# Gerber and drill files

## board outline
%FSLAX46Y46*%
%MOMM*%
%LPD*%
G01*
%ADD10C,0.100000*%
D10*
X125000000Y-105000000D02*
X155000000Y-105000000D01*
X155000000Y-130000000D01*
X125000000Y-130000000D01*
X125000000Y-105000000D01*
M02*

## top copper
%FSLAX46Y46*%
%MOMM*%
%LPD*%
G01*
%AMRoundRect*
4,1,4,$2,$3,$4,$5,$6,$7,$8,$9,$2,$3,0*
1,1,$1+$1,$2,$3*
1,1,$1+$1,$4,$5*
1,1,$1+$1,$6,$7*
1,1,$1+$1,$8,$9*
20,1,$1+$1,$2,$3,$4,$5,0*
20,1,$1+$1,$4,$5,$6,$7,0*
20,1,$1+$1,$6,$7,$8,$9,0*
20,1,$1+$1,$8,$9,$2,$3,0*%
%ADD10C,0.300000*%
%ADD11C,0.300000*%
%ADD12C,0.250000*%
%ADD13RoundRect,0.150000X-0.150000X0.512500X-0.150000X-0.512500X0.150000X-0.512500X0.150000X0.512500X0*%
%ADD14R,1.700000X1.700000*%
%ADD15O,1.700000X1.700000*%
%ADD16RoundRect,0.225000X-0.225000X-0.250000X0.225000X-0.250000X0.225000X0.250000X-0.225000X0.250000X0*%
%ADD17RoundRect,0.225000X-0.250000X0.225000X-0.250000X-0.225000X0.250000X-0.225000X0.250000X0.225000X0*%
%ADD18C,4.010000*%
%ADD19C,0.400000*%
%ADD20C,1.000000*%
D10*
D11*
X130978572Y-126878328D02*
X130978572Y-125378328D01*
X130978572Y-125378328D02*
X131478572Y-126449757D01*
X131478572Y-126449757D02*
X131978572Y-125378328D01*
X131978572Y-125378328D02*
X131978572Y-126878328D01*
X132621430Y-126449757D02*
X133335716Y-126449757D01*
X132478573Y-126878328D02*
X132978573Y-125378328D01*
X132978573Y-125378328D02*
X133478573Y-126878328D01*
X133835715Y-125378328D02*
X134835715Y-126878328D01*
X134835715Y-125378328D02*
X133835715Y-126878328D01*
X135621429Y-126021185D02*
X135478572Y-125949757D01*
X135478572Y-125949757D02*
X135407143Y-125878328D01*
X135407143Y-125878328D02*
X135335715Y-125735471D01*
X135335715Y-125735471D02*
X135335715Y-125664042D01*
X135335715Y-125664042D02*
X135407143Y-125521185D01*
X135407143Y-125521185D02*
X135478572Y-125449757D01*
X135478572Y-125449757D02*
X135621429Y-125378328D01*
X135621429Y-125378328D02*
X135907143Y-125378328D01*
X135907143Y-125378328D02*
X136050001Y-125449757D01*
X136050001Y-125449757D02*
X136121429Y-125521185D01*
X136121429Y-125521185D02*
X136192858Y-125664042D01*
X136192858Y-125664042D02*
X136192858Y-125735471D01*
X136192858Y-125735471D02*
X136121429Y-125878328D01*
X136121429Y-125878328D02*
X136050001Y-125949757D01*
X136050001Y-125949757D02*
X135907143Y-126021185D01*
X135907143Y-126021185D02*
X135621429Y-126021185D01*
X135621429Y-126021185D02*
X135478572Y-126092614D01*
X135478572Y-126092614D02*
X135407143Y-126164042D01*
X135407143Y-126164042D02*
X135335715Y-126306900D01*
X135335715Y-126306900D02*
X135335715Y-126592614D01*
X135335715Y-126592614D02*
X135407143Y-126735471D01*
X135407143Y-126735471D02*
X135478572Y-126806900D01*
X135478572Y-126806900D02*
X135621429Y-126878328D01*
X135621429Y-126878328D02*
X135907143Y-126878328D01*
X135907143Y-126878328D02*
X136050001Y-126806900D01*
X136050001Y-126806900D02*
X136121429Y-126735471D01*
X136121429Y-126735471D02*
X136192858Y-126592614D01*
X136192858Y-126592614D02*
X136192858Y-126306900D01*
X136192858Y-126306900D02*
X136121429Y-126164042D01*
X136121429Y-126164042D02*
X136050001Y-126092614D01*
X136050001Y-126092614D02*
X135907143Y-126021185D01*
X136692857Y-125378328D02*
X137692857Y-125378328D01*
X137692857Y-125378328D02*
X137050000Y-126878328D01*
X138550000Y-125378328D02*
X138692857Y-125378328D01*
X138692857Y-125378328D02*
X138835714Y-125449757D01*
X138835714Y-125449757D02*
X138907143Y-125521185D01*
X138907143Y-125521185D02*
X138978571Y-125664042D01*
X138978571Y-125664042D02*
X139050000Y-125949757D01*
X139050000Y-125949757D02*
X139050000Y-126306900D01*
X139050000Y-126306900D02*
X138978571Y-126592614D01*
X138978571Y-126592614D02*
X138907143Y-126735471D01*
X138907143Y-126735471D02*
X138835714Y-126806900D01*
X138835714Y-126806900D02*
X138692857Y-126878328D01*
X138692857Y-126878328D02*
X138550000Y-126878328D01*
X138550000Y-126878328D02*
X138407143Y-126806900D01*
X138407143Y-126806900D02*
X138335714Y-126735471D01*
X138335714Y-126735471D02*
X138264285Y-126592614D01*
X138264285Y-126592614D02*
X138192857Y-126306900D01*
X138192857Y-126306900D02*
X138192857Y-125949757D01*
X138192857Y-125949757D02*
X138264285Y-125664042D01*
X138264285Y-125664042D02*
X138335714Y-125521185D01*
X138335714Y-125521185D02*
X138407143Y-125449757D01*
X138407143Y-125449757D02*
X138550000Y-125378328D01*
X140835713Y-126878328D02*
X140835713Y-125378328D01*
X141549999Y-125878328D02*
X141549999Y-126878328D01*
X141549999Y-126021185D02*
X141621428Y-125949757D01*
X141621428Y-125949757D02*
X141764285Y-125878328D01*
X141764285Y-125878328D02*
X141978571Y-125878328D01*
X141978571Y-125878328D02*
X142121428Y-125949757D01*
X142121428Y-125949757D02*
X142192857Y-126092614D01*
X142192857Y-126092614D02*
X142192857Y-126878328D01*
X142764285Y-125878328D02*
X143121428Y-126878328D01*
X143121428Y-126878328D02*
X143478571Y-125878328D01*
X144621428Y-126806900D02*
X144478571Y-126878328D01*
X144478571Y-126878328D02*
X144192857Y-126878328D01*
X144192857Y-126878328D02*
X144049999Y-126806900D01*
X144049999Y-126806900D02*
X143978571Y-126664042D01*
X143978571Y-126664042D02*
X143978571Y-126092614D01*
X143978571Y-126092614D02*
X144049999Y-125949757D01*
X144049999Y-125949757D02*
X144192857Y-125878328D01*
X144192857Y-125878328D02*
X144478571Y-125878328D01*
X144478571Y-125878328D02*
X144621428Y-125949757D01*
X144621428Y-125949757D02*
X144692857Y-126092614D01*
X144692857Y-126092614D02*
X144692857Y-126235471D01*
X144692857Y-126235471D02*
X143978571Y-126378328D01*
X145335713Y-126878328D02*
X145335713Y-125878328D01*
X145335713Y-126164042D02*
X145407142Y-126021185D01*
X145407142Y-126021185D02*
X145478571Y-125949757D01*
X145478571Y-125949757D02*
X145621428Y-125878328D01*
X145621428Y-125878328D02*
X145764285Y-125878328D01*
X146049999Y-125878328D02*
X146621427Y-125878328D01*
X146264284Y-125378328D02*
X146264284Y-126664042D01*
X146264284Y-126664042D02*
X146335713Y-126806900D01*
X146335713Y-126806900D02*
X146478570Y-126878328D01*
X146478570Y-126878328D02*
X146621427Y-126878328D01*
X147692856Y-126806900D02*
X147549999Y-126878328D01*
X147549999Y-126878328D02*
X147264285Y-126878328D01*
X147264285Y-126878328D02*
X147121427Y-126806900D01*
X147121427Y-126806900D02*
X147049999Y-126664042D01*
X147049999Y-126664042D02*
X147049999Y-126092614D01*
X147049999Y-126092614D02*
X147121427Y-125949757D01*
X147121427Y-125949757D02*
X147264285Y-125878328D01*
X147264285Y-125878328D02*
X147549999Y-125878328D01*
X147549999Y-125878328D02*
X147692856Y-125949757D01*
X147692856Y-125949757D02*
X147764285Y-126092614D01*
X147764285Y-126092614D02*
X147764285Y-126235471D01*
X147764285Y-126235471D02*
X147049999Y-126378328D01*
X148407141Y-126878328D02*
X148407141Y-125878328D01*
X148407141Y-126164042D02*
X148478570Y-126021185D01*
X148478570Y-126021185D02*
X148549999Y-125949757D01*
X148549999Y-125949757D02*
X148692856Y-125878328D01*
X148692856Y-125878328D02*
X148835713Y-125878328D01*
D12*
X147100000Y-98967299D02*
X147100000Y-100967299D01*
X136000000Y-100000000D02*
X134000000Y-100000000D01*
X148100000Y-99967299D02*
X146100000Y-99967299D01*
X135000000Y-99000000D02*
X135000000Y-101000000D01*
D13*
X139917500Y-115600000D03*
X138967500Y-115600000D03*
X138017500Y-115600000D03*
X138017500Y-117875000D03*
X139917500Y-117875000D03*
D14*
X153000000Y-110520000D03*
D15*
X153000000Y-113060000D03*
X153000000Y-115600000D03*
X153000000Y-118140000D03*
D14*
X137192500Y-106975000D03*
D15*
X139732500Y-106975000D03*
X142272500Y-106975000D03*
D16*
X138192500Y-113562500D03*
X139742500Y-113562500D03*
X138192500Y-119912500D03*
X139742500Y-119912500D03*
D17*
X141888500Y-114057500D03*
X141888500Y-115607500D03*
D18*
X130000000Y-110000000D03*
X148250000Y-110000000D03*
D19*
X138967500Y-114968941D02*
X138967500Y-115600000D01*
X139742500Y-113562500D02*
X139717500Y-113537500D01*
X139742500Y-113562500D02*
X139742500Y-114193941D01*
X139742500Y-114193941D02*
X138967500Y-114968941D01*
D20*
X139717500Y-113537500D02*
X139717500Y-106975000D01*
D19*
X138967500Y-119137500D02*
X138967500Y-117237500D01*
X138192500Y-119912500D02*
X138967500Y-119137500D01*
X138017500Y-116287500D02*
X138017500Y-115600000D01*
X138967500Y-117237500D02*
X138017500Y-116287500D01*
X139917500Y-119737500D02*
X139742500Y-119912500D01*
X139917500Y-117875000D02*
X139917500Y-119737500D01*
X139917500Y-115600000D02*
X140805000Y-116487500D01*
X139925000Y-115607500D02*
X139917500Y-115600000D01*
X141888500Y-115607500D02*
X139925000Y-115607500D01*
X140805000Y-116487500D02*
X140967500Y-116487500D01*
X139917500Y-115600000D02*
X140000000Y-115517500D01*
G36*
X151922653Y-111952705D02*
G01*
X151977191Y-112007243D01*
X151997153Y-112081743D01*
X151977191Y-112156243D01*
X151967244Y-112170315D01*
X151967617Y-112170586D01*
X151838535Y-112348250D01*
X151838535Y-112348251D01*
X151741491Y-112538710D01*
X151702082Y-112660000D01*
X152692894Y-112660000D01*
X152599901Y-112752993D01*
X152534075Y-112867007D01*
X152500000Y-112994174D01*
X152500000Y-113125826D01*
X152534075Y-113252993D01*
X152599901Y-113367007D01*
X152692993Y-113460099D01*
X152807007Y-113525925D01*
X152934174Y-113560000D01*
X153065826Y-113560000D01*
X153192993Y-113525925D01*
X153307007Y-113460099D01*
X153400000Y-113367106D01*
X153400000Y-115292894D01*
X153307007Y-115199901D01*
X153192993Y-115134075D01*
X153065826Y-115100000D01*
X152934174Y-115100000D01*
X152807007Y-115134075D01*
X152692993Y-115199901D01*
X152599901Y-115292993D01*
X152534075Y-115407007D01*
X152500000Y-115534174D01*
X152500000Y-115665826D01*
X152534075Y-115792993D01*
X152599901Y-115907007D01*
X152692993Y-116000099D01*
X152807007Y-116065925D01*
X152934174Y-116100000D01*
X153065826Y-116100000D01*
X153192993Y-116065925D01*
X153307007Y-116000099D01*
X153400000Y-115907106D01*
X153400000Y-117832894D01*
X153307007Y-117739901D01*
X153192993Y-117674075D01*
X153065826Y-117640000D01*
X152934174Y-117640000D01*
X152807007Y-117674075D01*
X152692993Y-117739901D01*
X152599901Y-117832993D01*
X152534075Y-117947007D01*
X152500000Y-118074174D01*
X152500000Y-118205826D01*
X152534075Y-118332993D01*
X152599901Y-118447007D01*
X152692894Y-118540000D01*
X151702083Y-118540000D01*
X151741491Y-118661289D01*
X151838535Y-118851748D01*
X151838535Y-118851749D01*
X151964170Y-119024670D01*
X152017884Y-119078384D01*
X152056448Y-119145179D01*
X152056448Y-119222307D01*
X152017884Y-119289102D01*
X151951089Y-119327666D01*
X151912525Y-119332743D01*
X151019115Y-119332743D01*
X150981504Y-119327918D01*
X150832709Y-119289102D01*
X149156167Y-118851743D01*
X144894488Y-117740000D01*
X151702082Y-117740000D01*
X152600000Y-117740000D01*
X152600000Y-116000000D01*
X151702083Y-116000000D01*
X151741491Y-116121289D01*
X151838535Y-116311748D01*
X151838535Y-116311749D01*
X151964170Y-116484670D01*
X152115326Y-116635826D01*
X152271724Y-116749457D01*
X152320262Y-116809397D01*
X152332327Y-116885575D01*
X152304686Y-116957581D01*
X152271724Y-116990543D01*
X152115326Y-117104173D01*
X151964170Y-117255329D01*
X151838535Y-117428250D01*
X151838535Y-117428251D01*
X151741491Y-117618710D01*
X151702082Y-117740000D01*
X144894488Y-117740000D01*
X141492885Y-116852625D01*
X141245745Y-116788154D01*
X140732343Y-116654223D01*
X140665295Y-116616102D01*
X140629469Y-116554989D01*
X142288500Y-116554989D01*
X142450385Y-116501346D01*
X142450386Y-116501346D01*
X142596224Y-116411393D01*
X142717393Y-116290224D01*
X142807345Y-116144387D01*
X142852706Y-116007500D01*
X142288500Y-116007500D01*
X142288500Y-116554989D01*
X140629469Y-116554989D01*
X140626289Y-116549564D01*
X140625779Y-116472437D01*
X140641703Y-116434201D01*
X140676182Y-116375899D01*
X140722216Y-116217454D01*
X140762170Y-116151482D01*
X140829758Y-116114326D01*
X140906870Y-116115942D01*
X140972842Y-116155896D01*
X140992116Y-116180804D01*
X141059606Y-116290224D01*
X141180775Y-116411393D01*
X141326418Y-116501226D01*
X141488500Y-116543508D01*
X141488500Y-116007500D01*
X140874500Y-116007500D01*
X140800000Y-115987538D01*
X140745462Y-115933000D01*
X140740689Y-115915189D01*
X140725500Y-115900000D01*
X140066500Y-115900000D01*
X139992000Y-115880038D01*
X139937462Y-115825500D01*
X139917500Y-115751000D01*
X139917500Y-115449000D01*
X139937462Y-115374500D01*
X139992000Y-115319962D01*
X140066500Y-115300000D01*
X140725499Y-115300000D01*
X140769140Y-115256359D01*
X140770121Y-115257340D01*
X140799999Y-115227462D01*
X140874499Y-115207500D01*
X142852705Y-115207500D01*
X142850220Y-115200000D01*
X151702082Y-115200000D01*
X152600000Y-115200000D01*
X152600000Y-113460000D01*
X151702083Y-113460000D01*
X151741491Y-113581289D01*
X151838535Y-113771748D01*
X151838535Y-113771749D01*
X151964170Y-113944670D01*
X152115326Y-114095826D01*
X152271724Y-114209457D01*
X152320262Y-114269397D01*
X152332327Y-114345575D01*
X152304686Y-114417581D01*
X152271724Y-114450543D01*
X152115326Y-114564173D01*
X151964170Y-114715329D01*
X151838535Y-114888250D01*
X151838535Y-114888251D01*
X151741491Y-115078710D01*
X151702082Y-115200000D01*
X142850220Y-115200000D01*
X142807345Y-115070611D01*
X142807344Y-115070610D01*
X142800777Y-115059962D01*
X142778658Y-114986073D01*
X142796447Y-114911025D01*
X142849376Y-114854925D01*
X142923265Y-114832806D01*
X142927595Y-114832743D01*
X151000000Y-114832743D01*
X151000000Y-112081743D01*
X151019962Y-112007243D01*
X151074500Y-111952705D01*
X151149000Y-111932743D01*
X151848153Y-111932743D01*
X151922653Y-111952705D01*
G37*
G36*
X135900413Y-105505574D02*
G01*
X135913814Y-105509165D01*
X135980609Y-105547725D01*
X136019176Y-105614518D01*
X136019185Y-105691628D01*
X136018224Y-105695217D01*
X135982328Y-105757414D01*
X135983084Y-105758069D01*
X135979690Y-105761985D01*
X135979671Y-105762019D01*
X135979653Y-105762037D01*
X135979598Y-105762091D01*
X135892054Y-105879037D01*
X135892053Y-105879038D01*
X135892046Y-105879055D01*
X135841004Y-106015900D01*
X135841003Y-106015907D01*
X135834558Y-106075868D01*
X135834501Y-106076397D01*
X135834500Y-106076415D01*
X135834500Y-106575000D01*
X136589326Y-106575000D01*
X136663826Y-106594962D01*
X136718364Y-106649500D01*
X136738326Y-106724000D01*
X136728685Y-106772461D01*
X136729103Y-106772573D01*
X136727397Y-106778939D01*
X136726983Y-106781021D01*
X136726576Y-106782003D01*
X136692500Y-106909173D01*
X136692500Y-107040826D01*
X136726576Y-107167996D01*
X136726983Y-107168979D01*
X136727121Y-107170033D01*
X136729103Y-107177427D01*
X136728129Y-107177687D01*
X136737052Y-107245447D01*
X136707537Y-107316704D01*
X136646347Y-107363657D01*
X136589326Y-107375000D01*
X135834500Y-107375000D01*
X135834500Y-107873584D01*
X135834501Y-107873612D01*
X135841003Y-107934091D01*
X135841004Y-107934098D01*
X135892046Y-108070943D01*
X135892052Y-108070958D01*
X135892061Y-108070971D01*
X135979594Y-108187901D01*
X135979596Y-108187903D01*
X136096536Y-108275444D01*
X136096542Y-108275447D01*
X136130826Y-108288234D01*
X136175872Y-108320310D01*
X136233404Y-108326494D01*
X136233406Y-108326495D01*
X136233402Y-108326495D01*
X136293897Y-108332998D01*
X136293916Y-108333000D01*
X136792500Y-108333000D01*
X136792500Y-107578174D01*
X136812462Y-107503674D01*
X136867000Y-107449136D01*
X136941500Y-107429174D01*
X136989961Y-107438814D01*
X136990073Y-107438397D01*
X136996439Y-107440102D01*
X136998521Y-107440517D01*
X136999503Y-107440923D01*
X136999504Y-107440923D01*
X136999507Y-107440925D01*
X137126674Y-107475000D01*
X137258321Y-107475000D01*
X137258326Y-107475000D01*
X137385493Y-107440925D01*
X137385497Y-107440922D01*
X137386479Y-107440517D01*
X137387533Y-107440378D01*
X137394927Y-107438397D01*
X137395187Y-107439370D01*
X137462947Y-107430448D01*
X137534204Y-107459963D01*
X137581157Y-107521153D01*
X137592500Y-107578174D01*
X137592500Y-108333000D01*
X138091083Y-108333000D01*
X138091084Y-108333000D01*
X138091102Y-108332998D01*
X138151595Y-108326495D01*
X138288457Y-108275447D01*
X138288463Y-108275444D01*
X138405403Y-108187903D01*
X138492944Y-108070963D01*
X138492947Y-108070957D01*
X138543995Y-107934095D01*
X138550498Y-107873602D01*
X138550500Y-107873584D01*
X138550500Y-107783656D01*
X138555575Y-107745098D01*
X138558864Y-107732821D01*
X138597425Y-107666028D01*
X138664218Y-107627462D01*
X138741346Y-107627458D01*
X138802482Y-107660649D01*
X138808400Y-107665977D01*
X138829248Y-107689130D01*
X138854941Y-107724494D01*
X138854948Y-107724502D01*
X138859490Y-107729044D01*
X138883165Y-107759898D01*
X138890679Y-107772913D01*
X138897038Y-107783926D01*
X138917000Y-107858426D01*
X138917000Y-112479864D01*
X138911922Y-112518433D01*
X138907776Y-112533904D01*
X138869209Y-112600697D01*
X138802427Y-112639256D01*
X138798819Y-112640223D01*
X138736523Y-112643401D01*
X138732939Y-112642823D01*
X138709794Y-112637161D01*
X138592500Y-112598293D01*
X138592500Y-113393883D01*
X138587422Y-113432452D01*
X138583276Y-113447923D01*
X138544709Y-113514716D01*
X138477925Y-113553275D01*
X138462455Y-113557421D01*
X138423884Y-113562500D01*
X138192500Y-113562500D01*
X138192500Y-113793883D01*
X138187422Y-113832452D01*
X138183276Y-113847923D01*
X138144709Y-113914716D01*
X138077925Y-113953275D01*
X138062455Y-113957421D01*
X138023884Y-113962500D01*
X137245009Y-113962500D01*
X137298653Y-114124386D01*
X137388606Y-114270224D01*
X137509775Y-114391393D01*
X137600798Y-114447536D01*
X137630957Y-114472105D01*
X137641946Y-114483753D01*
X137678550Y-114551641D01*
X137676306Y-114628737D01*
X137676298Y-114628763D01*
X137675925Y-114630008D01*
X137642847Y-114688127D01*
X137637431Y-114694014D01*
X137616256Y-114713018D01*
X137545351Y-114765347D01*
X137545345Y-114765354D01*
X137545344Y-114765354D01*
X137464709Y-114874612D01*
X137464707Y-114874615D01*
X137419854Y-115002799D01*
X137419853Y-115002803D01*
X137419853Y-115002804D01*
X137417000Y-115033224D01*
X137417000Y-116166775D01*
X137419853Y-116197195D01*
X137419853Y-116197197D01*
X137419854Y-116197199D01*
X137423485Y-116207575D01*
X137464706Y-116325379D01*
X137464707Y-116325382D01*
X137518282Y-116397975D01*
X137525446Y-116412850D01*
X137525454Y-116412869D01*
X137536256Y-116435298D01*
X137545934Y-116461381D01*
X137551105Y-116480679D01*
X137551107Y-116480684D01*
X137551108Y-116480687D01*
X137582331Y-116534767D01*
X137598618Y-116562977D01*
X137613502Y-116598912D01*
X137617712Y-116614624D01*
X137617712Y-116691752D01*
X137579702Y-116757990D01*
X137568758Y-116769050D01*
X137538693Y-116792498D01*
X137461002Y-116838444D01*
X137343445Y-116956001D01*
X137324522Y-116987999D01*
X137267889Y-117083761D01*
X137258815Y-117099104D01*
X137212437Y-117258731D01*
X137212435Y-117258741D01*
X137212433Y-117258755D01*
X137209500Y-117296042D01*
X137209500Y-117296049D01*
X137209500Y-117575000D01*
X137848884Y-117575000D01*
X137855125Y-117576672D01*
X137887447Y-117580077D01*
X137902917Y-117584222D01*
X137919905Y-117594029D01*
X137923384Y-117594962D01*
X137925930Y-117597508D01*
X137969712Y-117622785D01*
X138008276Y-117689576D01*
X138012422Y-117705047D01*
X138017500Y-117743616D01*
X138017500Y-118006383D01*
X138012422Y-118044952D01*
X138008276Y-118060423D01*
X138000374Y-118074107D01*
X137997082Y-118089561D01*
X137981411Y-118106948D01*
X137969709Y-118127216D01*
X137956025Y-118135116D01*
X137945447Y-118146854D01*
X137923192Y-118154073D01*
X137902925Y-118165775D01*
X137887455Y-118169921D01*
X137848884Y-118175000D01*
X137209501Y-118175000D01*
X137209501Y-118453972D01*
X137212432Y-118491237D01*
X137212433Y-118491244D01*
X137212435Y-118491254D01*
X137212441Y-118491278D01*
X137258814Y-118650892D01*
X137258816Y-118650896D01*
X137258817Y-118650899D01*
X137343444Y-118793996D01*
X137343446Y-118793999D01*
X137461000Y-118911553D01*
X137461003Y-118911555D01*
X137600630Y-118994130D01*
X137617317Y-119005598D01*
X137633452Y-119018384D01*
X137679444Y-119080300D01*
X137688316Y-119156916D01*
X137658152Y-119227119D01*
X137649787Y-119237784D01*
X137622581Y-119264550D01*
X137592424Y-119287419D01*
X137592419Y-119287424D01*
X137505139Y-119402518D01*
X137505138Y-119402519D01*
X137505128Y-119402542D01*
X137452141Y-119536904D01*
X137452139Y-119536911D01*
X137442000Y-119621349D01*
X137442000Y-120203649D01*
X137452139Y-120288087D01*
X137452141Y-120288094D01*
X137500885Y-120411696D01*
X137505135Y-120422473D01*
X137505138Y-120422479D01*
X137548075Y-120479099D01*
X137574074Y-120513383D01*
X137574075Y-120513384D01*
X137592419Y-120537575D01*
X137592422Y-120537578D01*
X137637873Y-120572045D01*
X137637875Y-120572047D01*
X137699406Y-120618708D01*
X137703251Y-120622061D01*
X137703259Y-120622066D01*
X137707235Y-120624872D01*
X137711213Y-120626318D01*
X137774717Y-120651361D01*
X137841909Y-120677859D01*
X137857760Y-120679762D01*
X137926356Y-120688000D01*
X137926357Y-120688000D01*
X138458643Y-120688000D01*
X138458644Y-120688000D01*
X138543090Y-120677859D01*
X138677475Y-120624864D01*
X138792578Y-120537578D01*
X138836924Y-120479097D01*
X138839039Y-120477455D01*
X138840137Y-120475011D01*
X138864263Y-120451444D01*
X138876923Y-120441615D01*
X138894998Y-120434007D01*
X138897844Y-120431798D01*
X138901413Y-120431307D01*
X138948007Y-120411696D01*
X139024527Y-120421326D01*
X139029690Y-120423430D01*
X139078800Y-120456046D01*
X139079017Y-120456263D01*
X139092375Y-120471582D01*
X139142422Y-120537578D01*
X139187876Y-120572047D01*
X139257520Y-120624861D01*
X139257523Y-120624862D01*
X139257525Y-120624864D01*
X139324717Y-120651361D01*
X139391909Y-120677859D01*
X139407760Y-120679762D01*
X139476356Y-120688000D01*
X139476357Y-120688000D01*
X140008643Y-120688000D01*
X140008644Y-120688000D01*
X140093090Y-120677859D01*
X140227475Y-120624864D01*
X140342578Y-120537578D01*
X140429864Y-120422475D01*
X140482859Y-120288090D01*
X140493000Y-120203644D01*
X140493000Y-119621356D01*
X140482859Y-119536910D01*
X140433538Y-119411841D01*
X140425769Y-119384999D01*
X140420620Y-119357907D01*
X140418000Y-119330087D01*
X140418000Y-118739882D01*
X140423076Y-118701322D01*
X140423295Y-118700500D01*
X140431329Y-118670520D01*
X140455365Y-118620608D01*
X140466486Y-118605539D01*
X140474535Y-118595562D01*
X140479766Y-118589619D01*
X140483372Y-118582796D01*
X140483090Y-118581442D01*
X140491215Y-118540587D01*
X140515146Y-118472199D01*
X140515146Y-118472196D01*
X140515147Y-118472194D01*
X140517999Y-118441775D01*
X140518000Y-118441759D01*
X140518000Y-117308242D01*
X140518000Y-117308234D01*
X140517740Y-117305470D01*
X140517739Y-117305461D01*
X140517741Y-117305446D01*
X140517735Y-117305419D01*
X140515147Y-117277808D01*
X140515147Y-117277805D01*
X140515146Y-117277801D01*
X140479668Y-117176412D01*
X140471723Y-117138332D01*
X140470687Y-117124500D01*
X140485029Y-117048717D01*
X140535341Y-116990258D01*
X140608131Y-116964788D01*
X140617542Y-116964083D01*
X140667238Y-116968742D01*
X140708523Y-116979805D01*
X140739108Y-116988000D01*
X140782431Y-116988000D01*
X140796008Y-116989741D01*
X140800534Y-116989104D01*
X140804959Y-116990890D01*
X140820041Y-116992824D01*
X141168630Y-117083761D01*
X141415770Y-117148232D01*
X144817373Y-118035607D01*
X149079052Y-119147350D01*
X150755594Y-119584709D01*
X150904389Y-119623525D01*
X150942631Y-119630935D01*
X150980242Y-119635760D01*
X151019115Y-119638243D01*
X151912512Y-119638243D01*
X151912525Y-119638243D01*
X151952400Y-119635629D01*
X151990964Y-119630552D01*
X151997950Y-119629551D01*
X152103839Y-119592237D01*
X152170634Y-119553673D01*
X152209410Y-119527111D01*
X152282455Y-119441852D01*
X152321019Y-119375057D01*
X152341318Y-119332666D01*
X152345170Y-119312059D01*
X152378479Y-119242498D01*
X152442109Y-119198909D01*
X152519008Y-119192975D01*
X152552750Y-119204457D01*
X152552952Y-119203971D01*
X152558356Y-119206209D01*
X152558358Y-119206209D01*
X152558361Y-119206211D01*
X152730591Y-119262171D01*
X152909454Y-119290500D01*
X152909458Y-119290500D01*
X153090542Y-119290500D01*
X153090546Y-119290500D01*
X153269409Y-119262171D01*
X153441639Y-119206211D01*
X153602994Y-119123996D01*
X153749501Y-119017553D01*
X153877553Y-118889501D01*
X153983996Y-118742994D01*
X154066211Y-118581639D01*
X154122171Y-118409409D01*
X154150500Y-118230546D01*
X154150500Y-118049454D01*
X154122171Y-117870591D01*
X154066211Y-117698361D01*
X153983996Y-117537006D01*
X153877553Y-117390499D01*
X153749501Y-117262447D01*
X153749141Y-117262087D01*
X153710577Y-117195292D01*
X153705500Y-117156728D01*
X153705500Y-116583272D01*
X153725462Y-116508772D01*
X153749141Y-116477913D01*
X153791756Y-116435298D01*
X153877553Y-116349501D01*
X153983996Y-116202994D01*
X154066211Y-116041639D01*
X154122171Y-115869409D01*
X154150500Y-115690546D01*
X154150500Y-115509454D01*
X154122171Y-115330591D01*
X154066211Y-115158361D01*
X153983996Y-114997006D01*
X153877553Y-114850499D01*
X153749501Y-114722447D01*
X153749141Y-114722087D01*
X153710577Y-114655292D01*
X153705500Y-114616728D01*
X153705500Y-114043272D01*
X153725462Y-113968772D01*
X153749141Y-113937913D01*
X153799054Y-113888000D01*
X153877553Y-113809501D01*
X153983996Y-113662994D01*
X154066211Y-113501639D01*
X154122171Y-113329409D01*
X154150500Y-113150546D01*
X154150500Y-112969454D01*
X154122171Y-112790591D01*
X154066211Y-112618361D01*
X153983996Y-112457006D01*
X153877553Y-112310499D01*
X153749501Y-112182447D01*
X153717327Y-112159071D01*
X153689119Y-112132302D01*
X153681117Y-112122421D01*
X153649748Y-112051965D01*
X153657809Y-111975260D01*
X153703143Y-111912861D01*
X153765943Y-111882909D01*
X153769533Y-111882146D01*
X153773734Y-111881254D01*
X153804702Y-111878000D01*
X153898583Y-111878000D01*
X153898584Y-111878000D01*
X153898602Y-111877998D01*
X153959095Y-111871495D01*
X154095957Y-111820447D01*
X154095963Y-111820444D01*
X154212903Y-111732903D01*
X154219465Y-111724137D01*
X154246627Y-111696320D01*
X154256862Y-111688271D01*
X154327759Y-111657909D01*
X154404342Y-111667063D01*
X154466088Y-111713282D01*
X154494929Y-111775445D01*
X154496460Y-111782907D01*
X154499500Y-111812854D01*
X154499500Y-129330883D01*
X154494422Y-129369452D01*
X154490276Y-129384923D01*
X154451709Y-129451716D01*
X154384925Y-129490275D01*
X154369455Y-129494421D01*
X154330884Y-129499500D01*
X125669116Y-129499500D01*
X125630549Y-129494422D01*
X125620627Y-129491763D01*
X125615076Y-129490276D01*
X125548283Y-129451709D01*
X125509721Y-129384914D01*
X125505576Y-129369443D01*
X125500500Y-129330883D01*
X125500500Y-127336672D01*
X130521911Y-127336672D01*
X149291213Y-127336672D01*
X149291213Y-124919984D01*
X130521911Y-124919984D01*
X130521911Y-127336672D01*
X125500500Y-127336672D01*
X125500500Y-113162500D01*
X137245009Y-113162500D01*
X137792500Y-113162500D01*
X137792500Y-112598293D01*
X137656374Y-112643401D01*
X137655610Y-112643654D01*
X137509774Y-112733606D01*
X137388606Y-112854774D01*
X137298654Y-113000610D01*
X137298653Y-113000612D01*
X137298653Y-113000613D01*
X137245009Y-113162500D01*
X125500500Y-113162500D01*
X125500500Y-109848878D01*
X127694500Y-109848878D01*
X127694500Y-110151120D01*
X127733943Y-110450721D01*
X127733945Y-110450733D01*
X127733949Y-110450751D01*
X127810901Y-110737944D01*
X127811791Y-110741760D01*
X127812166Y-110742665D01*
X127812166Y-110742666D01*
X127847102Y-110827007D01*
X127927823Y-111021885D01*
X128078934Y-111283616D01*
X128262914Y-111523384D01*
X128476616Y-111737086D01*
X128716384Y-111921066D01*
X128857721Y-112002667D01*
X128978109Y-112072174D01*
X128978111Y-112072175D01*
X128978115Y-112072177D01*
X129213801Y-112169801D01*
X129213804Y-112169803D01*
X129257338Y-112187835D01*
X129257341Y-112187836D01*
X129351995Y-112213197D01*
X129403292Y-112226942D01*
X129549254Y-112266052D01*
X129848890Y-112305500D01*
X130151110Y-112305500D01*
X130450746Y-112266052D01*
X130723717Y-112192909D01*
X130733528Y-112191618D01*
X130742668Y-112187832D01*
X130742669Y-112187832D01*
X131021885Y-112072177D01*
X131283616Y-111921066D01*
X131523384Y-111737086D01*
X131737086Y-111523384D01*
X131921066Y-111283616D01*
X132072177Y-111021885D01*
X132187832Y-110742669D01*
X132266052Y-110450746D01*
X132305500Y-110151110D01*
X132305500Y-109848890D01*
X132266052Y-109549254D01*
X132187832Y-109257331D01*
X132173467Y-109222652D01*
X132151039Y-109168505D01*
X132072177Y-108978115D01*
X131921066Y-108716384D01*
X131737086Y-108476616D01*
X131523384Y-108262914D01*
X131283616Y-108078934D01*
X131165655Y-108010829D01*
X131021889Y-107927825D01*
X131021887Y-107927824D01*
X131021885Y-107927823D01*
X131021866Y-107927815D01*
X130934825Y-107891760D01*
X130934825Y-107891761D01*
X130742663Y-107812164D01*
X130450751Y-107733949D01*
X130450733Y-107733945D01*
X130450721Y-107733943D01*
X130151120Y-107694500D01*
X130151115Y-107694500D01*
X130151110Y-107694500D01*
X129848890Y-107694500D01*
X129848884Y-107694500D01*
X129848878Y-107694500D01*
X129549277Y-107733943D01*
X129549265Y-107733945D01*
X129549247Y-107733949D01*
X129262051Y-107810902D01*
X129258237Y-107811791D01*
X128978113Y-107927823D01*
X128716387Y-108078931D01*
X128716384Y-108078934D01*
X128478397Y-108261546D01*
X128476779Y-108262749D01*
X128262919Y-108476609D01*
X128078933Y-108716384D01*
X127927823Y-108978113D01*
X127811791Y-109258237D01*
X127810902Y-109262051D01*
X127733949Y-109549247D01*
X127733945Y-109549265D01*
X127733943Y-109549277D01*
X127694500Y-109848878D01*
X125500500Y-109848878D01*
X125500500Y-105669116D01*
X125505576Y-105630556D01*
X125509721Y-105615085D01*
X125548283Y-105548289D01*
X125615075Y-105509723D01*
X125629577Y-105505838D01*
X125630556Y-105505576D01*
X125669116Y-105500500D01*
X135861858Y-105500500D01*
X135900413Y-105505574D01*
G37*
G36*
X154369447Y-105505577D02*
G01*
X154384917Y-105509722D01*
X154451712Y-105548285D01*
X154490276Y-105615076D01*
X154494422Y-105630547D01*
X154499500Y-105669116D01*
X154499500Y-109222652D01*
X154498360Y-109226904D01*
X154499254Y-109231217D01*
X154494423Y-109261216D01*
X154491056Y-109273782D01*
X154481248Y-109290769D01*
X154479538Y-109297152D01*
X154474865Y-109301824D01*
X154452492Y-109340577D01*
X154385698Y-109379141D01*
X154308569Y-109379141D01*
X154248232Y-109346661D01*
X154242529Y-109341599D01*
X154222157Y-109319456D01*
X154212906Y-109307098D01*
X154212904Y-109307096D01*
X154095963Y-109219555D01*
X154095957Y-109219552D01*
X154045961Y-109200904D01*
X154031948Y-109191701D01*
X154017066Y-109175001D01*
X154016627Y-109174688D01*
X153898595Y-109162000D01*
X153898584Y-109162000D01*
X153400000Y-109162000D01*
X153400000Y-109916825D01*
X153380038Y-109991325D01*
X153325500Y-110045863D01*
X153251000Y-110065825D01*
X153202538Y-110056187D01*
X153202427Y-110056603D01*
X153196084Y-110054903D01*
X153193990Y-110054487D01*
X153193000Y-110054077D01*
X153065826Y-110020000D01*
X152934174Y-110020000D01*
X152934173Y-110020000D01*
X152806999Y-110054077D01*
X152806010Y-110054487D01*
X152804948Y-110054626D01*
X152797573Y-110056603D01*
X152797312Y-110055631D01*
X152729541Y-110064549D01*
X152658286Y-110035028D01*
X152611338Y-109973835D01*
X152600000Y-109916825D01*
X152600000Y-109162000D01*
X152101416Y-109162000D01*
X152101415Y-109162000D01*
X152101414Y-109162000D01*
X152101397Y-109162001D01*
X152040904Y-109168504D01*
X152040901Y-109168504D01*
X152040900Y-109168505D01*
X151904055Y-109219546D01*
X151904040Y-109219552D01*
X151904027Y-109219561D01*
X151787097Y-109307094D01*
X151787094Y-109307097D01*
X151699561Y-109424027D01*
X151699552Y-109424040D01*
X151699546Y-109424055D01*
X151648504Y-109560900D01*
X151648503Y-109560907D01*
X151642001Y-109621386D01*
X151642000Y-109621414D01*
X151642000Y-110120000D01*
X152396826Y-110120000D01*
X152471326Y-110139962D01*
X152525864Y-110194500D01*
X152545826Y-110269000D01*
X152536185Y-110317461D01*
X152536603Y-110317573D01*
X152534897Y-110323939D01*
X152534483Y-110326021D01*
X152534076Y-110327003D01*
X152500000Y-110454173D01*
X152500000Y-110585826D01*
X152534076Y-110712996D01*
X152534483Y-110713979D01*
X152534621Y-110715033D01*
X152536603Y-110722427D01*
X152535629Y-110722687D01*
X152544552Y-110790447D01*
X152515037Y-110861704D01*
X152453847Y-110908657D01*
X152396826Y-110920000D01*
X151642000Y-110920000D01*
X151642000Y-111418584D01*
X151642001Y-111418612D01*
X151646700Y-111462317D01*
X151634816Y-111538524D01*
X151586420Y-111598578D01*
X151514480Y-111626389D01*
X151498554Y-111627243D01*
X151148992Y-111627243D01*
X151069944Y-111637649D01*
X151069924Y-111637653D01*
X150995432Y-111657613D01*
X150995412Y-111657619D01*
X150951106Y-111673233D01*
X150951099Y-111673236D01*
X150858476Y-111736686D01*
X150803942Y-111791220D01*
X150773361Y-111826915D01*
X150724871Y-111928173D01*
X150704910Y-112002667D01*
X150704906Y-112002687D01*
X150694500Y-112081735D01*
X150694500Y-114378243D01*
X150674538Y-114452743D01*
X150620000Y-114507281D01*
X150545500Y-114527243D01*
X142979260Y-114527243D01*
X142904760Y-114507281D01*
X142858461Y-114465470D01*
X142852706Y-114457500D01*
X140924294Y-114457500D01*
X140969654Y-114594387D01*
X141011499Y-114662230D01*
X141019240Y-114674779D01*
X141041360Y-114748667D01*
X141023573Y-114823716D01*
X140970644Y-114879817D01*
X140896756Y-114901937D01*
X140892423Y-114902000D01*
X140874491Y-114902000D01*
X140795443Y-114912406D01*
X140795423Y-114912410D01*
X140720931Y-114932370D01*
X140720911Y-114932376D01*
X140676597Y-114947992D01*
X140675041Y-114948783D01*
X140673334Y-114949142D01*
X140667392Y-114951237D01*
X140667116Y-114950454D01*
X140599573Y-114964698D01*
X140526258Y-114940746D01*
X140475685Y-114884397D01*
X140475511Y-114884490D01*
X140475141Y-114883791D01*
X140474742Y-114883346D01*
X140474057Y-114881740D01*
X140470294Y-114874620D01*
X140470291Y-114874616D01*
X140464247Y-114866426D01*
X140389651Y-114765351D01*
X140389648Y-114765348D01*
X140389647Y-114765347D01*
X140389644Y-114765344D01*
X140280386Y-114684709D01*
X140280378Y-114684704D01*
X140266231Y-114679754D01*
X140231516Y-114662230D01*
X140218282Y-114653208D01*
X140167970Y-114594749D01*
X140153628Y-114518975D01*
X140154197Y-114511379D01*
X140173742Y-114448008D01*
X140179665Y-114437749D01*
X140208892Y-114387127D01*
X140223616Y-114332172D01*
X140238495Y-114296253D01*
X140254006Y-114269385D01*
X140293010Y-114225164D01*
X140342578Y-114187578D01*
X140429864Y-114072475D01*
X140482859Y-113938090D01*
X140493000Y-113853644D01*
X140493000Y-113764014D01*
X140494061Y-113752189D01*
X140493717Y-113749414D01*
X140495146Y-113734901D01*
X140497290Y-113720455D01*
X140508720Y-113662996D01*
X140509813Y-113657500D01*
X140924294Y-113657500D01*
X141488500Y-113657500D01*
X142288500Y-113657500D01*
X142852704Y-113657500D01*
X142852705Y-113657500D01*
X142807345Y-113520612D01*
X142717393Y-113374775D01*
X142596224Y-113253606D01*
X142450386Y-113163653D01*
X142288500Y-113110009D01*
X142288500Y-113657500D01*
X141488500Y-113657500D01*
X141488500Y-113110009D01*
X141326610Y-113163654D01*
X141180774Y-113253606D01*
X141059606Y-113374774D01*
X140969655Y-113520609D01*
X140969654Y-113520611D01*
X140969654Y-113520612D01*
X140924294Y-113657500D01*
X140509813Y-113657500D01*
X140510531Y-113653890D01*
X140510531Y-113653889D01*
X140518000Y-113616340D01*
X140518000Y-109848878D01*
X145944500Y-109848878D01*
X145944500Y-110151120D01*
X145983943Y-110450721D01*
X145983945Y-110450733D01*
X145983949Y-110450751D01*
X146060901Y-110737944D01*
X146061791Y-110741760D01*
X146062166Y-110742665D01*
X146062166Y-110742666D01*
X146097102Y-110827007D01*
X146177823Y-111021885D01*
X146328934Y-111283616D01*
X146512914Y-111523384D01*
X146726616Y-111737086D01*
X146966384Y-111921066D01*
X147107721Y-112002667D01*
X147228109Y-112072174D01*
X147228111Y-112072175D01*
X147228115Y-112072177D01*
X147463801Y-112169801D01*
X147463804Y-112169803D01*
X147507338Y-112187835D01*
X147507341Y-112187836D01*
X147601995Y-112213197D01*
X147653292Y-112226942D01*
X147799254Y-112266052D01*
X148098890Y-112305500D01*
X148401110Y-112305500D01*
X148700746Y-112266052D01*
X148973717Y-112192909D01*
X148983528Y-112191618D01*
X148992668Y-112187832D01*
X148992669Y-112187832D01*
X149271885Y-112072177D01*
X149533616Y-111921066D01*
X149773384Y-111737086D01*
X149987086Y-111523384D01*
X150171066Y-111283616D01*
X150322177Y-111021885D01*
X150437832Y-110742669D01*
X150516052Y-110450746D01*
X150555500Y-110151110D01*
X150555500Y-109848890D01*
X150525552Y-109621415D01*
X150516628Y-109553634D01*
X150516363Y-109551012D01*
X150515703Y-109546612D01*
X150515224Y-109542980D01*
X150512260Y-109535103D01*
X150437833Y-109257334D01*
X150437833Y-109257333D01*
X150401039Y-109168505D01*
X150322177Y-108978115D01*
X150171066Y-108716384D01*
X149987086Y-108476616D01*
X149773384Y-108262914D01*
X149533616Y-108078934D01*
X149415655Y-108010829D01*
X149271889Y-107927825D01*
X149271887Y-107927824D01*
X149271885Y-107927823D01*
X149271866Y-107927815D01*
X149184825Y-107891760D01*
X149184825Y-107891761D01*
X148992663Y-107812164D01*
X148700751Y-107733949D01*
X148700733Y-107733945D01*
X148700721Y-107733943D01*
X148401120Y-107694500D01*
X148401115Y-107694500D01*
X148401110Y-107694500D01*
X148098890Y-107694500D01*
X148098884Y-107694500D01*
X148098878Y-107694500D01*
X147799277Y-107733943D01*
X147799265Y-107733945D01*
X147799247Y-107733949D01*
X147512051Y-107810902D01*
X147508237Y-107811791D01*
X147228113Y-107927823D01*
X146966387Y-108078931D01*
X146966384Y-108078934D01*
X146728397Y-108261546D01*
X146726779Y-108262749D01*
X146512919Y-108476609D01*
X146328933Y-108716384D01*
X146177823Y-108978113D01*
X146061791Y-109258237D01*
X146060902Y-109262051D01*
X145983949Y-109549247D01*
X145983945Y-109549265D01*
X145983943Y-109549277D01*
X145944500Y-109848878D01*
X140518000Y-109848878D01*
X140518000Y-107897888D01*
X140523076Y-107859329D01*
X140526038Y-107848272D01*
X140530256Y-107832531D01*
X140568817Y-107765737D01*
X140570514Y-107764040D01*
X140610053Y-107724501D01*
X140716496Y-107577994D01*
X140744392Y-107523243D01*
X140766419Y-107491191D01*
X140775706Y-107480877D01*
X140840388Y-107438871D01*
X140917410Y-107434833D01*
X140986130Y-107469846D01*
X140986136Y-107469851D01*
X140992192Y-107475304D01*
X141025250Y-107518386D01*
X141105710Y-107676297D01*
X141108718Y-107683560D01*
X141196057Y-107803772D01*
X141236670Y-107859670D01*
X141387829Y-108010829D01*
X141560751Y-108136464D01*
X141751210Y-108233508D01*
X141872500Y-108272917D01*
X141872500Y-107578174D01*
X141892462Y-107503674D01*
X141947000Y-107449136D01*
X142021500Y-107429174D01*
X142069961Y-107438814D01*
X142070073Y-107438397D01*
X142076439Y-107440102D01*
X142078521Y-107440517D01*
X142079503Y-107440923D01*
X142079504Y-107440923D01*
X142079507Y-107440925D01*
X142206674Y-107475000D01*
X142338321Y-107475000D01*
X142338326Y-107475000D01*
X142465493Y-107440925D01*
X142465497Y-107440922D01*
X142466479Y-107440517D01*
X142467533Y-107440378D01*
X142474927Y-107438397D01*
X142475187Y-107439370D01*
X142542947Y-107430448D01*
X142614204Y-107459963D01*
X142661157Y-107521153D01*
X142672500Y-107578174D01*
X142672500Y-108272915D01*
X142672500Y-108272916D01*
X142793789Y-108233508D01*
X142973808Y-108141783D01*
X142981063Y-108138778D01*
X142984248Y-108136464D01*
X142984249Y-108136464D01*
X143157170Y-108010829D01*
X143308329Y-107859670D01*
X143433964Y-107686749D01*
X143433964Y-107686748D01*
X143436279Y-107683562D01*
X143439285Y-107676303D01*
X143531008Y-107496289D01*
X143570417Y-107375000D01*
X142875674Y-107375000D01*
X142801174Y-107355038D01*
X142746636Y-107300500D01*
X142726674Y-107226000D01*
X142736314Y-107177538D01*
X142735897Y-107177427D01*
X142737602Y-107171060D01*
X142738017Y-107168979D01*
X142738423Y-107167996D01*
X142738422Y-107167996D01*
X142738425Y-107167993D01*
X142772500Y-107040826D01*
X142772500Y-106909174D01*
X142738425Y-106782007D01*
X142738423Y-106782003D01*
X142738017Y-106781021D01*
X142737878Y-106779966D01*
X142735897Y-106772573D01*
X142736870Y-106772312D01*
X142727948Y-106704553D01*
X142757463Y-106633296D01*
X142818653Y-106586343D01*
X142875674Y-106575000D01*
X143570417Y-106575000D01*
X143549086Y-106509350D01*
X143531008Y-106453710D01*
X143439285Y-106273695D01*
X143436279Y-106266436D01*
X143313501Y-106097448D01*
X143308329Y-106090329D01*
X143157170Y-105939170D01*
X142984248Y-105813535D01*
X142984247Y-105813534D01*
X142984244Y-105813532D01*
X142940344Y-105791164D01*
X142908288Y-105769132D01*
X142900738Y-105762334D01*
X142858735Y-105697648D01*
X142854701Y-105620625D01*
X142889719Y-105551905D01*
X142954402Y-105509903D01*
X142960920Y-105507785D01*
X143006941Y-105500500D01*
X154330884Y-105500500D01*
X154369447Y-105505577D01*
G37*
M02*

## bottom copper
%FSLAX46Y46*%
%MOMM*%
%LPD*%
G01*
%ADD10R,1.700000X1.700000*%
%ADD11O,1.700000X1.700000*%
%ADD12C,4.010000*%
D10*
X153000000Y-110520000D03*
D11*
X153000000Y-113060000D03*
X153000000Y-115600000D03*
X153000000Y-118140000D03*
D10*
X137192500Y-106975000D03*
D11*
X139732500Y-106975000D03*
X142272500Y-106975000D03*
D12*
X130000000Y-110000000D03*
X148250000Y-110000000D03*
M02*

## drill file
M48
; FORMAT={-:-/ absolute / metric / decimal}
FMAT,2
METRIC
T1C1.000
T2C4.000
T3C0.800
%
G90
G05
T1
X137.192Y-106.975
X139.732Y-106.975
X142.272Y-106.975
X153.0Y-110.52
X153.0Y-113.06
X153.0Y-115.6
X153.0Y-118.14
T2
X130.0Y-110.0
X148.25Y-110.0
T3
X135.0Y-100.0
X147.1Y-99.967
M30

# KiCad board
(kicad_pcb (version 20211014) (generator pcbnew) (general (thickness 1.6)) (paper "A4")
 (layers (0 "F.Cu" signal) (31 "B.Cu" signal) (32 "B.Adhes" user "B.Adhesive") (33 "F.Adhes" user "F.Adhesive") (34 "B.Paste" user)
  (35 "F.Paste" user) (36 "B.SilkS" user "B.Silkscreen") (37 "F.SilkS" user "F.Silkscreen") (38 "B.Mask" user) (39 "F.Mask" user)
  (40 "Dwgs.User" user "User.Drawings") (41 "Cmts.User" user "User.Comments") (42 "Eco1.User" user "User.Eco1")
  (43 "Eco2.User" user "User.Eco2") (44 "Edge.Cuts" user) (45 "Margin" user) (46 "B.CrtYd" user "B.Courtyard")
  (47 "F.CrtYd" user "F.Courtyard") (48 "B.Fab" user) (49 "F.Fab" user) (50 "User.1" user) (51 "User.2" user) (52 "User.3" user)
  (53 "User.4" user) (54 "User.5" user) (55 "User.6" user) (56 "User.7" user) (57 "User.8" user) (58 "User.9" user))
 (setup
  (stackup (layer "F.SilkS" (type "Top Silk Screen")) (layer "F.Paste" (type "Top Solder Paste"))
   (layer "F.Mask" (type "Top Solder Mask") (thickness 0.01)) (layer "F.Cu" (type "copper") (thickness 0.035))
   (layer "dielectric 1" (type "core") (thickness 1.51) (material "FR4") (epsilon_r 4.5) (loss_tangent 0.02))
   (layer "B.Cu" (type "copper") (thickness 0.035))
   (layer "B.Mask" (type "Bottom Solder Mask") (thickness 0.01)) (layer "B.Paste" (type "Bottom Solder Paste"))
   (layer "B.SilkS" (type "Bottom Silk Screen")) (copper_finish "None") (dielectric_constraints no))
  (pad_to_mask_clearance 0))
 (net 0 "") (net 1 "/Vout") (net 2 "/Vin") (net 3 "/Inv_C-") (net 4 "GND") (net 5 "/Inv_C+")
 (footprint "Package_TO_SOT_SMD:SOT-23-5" (layer "F.Cu") (at 138.9675 116.7375 -90) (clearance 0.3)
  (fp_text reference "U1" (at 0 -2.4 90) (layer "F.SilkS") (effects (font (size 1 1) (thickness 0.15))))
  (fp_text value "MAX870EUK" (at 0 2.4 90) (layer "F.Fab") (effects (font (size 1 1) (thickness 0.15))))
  (pad "1" smd roundrect (at -1.1375 -0.95 270) (size 1.325 0.6) (layers "F.Cu" "F.Paste" "F.Mask") (roundrect_rratio 0.25) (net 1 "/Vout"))
  (pad "2" smd roundrect (at -1.1375 0 270) (size 1.325 0.6) (layers "F.Cu" "F.Paste" "F.Mask") (roundrect_rratio 0.25) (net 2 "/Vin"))
  (pad "3" smd roundrect (at -1.1375 0.95 270) (size 1.325 0.6) (layers "F.Cu" "F.Paste" "F.Mask") (roundrect_rratio 0.25) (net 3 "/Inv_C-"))
  (pad "4" smd roundrect (at 1.1375 0.95 270) (size 1.325 0.6) (layers "F.Cu" "F.Paste" "F.Mask") (roundrect_rratio 0.25) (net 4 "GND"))
  (pad "5" smd roundrect (at 1.1375 -0.95 270) (size 1.325 0.6) (layers "F.Cu" "F.Paste" "F.Mask") (roundrect_rratio 0.25) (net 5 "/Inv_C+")))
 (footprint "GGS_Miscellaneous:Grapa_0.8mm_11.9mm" (layer "F.Cu") (at 135 100)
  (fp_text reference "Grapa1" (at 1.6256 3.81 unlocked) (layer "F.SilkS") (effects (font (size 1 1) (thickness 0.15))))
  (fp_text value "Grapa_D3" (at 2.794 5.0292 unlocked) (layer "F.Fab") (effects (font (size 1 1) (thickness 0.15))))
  (fp_line (start 12.1 -1.032701) (end 12.1 0.967299) (layer "F.Cu") (width 0.25))
  (fp_line (start 1 0) (end -1 0) (layer "F.Cu") (width 0.25))
  (fp_line (start 13.1 -0.032701) (end 11.1 -0.032701) (layer "F.Cu") (width 0.25))
  (fp_line (start 0 -1) (end 0 1) (layer "F.Cu") (width 0.25))
  (pad "" np_thru_hole circle (at 12.1 -0.032701) (size 0.8 0.8) (drill 0.8) (layers F&B.Cu *.Mask))
  (pad "" np_thru_hole circle (at 0 0) (size 0.8 0.8) (drill 0.8) (layers F&B.Cu *.Mask)))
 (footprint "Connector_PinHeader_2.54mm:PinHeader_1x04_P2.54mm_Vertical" (layer "F.Cu") (at 153 110.52)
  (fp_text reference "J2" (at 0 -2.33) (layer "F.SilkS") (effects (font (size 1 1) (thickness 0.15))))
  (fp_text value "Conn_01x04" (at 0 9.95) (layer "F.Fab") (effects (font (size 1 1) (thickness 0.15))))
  (pad "1" thru_hole rect (at 0 0) (size 1.7 1.7) (drill 1) (layers *.Cu *.Mask) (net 4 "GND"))
  (pad "2" thru_hole oval (at 0 2.54) (size 1.7 1.7) (drill 1) (layers *.Cu *.Mask) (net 1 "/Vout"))
  (pad "3" thru_hole oval (at 0 5.08) (size 1.7 1.7) (drill 1) (layers *.Cu *.Mask) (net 1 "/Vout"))
  (pad "4" thru_hole oval (at 0 7.62) (size 1.7 1.7) (drill 1) (layers *.Cu *.Mask) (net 1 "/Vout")))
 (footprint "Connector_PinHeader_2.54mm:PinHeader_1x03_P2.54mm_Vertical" (layer "F.Cu") (at 137.1925 106.975 90)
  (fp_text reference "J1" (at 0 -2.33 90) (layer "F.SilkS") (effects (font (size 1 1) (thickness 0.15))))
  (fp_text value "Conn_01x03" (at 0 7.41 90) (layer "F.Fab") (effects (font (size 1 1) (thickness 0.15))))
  (pad "1" thru_hole rect (at 0 0 90) (size 1.7 1.7) (drill 1) (layers *.Cu *.Mask) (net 4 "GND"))
  (pad "2" thru_hole oval (at 0 2.54 90) (size 1.7 1.7) (drill 1) (layers *.Cu *.Mask) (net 2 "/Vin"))
  (pad "3" thru_hole oval (at 0 5.08 90) (size 1.7 1.7) (drill 1) (layers *.Cu *.Mask) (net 4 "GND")))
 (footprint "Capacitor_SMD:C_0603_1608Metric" (layer "F.Cu") (at 138.9675 113.5625)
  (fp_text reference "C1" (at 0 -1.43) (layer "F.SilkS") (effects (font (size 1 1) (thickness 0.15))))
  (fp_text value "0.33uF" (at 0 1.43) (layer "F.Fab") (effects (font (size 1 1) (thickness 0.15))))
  (pad "1" smd roundrect (at -0.775 0) (size 0.9 0.95) (layers "F.Cu" "F.Paste" "F.Mask") (roundrect_rratio 0.25) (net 4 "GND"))
  (pad "2" smd roundrect (at 0.775 0) (size 0.9 0.95) (layers "F.Cu" "F.Paste" "F.Mask") (roundrect_rratio 0.25) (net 2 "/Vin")))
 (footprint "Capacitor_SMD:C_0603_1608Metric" (layer "F.Cu") (at 138.9675 119.9125)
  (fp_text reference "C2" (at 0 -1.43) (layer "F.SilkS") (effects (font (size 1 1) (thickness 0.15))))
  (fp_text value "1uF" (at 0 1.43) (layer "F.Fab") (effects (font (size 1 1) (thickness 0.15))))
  (pad "1" smd roundrect (at -0.775 0) (size 0.9 0.95) (layers "F.Cu" "F.Paste" "F.Mask") (roundrect_rratio 0.25) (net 3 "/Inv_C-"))
  (pad "2" smd roundrect (at 0.775 0) (size 0.9 0.95) (layers "F.Cu" "F.Paste" "F.Mask") (roundrect_rratio 0.25) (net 5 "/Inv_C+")))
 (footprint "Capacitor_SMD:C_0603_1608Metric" (layer "F.Cu") (at 141.8885 114.8325 -90)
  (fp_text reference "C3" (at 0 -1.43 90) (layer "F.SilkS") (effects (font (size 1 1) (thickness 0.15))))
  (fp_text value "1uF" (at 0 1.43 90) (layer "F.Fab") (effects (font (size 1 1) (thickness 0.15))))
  (pad "1" smd roundrect (at -0.775 0 270) (size 0.9 0.95) (layers "F.Cu" "F.Paste" "F.Mask") (roundrect_rratio 0.25) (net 4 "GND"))
  (pad "2" smd roundrect (at 0.775 0 270) (size 0.9 0.95) (layers "F.Cu" "F.Paste" "F.Mask") (roundrect_rratio 0.25) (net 1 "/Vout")))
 (gr_rect (start 125 105) (end 155 130) (layer "Edge.Cuts") (width 0.1) (fill none))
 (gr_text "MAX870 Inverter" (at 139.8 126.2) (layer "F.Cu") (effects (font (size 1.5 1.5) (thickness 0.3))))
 (via (at 130 110) (size 4.01) (drill 4) (layers "F.Cu" "B.Cu") (free) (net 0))
 (via (at 148.25 110) (size 4.01) (drill 4) (layers "F.Cu" "B.Cu") (free) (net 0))
 (segment (start 138.9675 114.968941) (end 138.9675 115.6) (width 0.4) (layer "F.Cu") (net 2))
 (segment (start 139.7425 113.5625) (end 139.7175 113.5375) (width 0.4) (layer "F.Cu") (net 2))
 (segment (start 139.7425 113.5625) (end 139.7425 114.193941) (width 0.4) (layer "F.Cu") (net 2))
 (segment (start 139.7425 114.193941) (end 138.9675 114.968941) (width 0.4) (layer "F.Cu") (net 2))
 (segment (start 139.7175 113.5375) (end 139.7175 106.975) (width 1) (layer "F.Cu") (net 2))
 (segment (start 138.9675 119.1375) (end 138.9675 117.2375) (width 0.4) (layer "F.Cu") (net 3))
 (segment (start 138.1925 119.9125) (end 138.9675 119.1375) (width 0.4) (layer "F.Cu") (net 3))
 (segment (start 138.0175 116.2875) (end 138.0175 115.6) (width 0.4) (layer "F.Cu") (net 3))
 (segment (start 138.9675 117.2375) (end 138.0175 116.2875) (width 0.4) (layer "F.Cu") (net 3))
 (segment (start 139.9175 119.7375) (end 139.7425 119.9125) (width 0.4) (layer "F.Cu") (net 5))
 (segment (start 139.9175 117.875) (end 139.9175 119.7375) (width 0.4) (layer "F.Cu") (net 5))
 (segment (start 139.9175 115.6) (end 140.805 116.4875) (width 0.4) (layer "F.Cu") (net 1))
 (segment (start 139.925 115.6075) (end 139.9175 115.6) (width 0.4) (layer "F.Cu") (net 1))
 (segment (start 141.8885 115.6075) (end 139.925 115.6075) (width 0.4) (layer "F.Cu") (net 1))
 (segment (start 140.805 116.4875) (end 140.9675 116.4875) (width 0.4) (layer "F.Cu") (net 1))
 (segment (start 139.9175 115.6) (end 140 115.5175) (width 0.4) (layer "F.Cu") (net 1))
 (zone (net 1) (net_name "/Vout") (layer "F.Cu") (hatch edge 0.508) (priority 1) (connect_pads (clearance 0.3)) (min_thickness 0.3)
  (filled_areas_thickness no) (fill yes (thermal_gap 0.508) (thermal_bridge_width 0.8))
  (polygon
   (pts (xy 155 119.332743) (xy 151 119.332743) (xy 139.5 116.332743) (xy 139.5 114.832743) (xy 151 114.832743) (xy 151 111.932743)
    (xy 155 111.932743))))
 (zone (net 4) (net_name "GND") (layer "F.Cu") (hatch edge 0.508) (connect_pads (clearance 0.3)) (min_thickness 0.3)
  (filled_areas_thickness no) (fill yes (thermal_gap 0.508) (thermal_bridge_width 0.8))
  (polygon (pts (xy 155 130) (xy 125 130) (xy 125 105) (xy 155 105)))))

